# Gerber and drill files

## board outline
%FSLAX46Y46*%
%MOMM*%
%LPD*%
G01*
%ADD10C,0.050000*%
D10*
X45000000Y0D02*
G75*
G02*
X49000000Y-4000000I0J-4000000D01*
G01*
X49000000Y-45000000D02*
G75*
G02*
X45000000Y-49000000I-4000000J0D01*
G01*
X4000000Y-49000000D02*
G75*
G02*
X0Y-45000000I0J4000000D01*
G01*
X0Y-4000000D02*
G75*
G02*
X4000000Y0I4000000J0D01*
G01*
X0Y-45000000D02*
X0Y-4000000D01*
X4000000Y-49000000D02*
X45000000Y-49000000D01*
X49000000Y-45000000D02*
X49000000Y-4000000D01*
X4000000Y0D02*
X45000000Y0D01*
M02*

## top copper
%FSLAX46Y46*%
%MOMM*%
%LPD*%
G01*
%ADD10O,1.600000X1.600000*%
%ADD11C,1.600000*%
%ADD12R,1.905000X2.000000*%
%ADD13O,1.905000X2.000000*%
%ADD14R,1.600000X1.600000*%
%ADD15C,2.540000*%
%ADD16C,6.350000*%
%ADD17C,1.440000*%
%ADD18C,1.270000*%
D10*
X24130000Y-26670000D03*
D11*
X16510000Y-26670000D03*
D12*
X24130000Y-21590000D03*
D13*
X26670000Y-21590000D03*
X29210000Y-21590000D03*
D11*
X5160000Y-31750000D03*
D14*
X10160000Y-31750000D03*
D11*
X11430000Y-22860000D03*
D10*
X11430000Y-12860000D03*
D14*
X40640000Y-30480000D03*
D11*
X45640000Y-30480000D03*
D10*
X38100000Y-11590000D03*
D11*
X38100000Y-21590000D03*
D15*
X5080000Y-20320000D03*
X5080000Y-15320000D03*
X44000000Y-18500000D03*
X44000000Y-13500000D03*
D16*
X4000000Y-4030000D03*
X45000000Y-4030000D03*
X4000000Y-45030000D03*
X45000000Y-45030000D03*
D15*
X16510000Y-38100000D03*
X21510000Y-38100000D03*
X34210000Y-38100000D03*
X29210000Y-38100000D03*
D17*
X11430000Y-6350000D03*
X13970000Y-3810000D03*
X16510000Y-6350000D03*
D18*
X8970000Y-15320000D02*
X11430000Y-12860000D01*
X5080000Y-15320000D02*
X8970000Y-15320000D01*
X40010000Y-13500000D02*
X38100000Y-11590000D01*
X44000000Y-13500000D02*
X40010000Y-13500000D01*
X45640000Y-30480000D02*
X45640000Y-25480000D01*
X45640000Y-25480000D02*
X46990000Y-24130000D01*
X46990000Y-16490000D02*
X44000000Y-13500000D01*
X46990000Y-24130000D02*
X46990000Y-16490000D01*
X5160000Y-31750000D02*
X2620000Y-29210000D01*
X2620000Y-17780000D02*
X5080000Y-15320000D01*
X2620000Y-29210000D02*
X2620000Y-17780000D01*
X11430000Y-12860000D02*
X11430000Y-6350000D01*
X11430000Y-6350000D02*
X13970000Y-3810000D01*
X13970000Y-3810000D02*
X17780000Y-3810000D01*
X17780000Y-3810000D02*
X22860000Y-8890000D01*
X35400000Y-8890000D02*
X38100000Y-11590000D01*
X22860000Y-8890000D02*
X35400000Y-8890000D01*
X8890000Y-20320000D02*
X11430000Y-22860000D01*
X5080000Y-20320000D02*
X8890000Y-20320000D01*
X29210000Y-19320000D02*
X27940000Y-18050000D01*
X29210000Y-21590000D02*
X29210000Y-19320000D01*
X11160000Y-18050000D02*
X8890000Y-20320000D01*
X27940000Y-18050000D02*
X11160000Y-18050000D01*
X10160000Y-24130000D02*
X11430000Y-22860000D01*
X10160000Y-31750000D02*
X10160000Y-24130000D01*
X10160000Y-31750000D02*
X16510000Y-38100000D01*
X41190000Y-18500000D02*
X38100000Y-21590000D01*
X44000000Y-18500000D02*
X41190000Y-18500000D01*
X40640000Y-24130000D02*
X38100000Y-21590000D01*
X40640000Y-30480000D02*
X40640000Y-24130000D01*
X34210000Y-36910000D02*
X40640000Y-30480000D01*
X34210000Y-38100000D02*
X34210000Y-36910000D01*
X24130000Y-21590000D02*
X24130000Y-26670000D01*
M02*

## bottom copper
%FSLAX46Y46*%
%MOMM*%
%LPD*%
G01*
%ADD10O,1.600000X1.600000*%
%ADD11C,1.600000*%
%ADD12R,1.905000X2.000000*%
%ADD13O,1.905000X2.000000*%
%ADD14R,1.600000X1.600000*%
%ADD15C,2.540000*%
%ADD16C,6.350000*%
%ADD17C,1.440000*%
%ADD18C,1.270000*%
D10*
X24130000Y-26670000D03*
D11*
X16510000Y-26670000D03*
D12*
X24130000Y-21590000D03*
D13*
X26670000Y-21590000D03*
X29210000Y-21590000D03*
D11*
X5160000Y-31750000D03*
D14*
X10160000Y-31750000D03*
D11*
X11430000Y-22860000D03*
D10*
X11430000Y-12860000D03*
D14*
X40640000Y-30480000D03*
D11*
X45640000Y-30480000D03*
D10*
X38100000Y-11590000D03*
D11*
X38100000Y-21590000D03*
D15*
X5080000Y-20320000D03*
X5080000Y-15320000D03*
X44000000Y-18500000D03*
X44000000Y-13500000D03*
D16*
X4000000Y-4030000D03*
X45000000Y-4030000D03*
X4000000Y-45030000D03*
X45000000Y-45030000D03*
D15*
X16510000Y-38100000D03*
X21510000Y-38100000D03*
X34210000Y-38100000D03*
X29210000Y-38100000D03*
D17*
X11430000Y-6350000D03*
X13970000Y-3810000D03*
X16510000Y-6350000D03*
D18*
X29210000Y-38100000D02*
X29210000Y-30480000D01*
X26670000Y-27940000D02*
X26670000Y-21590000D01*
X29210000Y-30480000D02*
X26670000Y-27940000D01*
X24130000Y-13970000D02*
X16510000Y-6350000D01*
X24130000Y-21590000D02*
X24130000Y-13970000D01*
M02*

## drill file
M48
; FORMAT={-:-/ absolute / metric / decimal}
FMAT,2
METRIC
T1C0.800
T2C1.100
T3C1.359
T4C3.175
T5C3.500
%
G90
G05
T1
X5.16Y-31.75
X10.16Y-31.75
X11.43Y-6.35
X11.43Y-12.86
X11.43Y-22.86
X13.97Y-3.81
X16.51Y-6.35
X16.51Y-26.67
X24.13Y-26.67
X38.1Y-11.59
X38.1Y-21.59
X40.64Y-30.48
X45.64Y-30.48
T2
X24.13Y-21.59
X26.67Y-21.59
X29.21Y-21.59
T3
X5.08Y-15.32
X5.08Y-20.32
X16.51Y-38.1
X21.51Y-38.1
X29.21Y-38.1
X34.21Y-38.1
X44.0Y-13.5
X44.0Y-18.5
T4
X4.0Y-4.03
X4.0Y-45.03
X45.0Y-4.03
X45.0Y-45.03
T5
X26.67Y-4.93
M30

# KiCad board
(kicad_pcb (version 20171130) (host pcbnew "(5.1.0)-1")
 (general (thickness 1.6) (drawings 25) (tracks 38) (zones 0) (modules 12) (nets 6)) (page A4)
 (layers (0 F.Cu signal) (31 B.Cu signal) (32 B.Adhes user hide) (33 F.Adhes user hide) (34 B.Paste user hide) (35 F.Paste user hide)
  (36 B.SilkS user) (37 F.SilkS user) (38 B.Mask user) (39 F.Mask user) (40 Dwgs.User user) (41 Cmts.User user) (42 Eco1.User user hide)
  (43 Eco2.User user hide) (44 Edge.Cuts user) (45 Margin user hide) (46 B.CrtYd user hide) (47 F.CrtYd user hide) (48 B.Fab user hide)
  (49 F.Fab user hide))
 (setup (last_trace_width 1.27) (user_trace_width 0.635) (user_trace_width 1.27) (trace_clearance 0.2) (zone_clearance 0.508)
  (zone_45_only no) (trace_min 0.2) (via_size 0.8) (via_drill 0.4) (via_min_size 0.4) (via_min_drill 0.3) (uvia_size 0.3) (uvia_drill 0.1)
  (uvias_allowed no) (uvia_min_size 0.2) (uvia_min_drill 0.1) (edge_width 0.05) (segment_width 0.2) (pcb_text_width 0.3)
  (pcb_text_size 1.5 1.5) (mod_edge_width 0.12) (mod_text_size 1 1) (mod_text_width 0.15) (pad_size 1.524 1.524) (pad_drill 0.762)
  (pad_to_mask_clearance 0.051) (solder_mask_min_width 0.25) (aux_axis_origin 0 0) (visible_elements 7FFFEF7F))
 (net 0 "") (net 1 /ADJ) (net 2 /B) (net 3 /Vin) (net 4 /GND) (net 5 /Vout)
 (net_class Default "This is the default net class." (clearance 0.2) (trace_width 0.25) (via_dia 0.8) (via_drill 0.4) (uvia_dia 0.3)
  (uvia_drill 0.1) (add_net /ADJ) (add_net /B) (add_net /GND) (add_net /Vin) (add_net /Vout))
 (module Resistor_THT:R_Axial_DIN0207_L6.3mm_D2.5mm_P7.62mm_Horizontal (layer F.Cu) (at 16.51 26.67)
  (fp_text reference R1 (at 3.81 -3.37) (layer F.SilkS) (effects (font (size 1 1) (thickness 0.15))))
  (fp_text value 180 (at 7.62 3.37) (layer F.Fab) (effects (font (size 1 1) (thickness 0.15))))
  (pad 2 thru_hole oval (at 7.62 0) (size 1.6 1.6) (drill 0.8) (layers *.Cu *.Mask) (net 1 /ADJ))
  (pad 1 thru_hole circle (at 0 0) (size 1.6 1.6) (drill 0.8) (layers *.Cu *.Mask) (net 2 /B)))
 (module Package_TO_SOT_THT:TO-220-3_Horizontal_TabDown (layer F.Cu) (at 24.13 21.59)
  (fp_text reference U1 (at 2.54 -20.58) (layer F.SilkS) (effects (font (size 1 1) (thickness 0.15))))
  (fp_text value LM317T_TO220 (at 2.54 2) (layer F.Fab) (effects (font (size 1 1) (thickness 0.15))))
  (pad "" np_thru_hole oval (at 2.54 -16.66) (size 3.5 3.5) (drill 3.5) (layers *.Cu *.Mask))
  (pad 1 thru_hole rect (at 0 0) (size 1.905 2) (drill 1.1) (layers *.Cu *.Mask) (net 1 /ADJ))
  (pad 2 thru_hole oval (at 2.54 0) (size 1.905 2) (drill 1.1) (layers *.Cu *.Mask) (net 2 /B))
  (pad 3 thru_hole oval (at 5.08 0) (size 1.905 2) (drill 1.1) (layers *.Cu *.Mask) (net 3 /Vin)))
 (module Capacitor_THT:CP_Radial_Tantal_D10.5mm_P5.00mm (layer F.Cu) (at 10.16 31.75 180)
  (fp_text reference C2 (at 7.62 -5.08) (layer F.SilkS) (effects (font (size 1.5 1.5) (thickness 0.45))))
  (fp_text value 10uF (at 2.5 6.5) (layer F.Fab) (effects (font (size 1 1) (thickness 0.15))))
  (pad 2 thru_hole circle (at 5 0 180) (size 1.6 1.6) (drill 0.8) (layers *.Cu *.Mask) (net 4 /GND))
  (pad 1 thru_hole rect (at 0 0 180) (size 1.6 1.6) (drill 0.8) (layers *.Cu *.Mask) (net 3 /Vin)))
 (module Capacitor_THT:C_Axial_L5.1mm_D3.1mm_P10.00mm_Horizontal (layer F.Cu) (at 11.43 22.86 90)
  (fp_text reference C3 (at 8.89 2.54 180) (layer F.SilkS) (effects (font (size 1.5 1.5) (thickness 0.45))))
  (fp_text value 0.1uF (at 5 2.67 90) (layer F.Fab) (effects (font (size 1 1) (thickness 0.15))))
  (pad 1 thru_hole circle (at 0 0 90) (size 1.6 1.6) (drill 0.8) (layers *.Cu *.Mask) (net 3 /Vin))
  (pad 2 thru_hole oval (at 10 0 90) (size 1.6 1.6) (drill 0.8) (layers *.Cu *.Mask) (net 4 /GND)))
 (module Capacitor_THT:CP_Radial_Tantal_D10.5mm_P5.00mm (layer F.Cu) (at 40.64 30.48)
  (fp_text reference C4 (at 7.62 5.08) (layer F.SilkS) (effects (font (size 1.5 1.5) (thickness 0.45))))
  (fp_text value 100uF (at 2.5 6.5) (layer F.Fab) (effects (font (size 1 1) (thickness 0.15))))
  (pad 1 thru_hole rect (at 0 0) (size 1.6 1.6) (drill 0.8) (layers *.Cu *.Mask) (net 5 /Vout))
  (pad 2 thru_hole circle (at 5 0) (size 1.6 1.6) (drill 0.8) (layers *.Cu *.Mask) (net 4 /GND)))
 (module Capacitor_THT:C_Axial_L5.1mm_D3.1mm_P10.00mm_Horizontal (layer F.Cu) (at 38.1 21.59 90)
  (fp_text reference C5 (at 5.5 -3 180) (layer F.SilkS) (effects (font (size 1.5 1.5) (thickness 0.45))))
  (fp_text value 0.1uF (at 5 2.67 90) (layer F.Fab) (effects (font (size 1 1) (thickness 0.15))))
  (pad 2 thru_hole oval (at 10 0 90) (size 1.6 1.6) (drill 0.8) (layers *.Cu *.Mask) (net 4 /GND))
  (pad 1 thru_hole circle (at 0 0 90) (size 1.6 1.6) (drill 0.8) (layers *.Cu *.Mask) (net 5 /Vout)))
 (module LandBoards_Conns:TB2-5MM (layer F.Cu) (at 5.08 20.32 90)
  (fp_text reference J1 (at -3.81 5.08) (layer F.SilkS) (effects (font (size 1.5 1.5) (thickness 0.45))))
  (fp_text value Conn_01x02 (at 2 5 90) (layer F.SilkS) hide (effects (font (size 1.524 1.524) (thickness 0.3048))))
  (pad 1 thru_hole circle (at 0 0 90) (size 2.54 2.54) (drill 1.3589) (layers *.Cu *.Mask F.SilkS) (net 3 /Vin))
  (pad 2 thru_hole circle (at 5 0 90) (size 2.54 2.54) (drill 1.3589) (layers *.Cu *.Mask F.SilkS) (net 4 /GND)))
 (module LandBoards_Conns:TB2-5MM (layer F.Cu) (at 44 13.5 270)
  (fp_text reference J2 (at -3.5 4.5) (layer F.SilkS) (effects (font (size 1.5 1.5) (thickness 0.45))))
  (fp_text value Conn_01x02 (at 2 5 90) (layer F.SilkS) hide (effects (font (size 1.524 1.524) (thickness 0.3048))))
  (pad 2 thru_hole circle (at 5 0 270) (size 2.54 2.54) (drill 1.3589) (layers *.Cu *.Mask F.SilkS) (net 5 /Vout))
  (pad 1 thru_hole circle (at 0 0 270) (size 2.54 2.54) (drill 1.3589) (layers *.Cu *.Mask F.SilkS) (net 4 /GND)))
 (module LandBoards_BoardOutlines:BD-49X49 (layer F.Cu) (at 0 49.03)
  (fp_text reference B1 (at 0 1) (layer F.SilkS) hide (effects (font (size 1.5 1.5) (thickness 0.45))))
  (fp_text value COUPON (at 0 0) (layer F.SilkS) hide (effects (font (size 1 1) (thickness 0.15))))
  (pad 1 thru_hole circle (at 4 -45) (size 6.35 6.35) (drill 3.175) (layers *.Cu *.Mask F.SilkS))
  (pad 2 thru_hole circle (at 45 -45) (size 6.35 6.35) (drill 3.175) (layers *.Cu *.Mask F.SilkS))
  (pad 3 thru_hole circle (at 4 -4) (size 6.35 6.35) (drill 3.175) (layers *.Cu *.Mask F.SilkS))
  (pad 4 thru_hole circle (at 45 -4) (size 6.35 6.35) (drill 3.175) (layers *.Cu *.Mask F.SilkS)))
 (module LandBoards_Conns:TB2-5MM (layer F.Cu) (at 16.51 38.1)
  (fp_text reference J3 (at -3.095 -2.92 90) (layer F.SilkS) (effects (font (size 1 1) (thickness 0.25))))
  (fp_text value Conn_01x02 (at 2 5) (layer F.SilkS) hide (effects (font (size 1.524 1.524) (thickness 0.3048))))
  (pad 1 thru_hole circle (at 0 0) (size 2.54 2.54) (drill 1.3589) (layers *.Cu *.Mask F.SilkS) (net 3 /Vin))
  (pad 2 thru_hole circle (at 5 0) (size 2.54 2.54) (drill 1.3589) (layers *.Cu *.Mask F.SilkS)))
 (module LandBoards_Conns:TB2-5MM (layer F.Cu) (at 29.21 38.1)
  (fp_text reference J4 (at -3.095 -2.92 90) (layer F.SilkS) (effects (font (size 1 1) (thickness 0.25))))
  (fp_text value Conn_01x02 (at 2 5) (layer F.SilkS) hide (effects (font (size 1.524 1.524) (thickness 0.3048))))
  (pad 2 thru_hole circle (at 5 0) (size 2.54 2.54) (drill 1.3589) (layers *.Cu *.Mask F.SilkS) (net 5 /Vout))
  (pad 1 thru_hole circle (at 0 0) (size 2.54 2.54) (drill 1.3589) (layers *.Cu *.Mask F.SilkS) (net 2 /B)))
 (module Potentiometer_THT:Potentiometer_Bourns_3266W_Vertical (layer F.Cu) (at 11.43 6.35 180)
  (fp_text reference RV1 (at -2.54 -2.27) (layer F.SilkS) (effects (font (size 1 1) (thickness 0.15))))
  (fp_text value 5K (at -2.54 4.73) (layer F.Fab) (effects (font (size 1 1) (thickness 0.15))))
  (pad 1 thru_hole circle (at 0 0 180) (size 1.44 1.44) (drill 0.8) (layers *.Cu *.Mask) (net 4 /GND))
  (pad 2 thru_hole circle (at -2.54 2.54 180) (size 1.44 1.44) (drill 0.8) (layers *.Cu *.Mask) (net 4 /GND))
  (pad 3 thru_hole circle (at -5.08 0 180) (size 1.44 1.44) (drill 0.8) (layers *.Cu *.Mask) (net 1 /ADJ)))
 (gr_arc (start 45 4) (end 49 4) (angle -90) (layer Edge.Cuts) (width 0.05))
 (gr_arc (start 45 45) (end 45 49) (angle -90) (layer Edge.Cuts) (width 0.05))
 (gr_arc (start 4 45) (end 0 45) (angle -90) (layer Edge.Cuts) (width 0.05))
 (gr_arc (start 4 4) (end 4 0) (angle -90) (layer Edge.Cuts) (width 0.05))
 (gr_line (start 0 45) (end 0 4) (layer Edge.Cuts) (width 0.05))
 (gr_line (start 4 49) (end 45 49) (layer Edge.Cuts) (width 0.05))
 (gr_line (start 49 45) (end 49 4) (layer Edge.Cuts) (width 0.05))
 (gr_line (start 4 0) (end 45 0) (layer Edge.Cuts) (width 0.05))
 (segment (start 8.97 15.32) (end 11.43 12.86) (width 1.27) (layer F.Cu) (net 4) (status 20))
 (segment (start 5.08 15.32) (end 8.97 15.32) (width 1.27) (layer F.Cu) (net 4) (status 10))
 (segment (start 40.01 13.5) (end 38.1 11.59) (width 1.27) (layer F.Cu) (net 4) (status 20))
 (segment (start 44 13.5) (end 40.01 13.5) (width 1.27) (layer F.Cu) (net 4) (status 10))
 (segment (start 45.64 30.48) (end 45.64 25.48) (width 1.27) (layer F.Cu) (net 4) (status 10))
 (segment (start 45.64 25.48) (end 46.99 24.13) (width 1.27) (layer F.Cu) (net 4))
 (segment (start 46.99 16.49) (end 44 13.5) (width 1.27) (layer F.Cu) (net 4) (status 20))
 (segment (start 46.99 24.13) (end 46.99 16.49) (width 1.27) (layer F.Cu) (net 4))
 (segment (start 5.16 31.75) (end 2.62 29.21) (width 1.27) (layer F.Cu) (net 4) (status 10))
 (segment (start 2.62 17.78) (end 5.08 15.32) (width 1.27) (layer F.Cu) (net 4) (status 20))
 (segment (start 2.62 29.21) (end 2.62 17.78) (width 1.27) (layer F.Cu) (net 4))
 (segment (start 11.43 12.86) (end 11.43 6.35) (width 1.27) (layer F.Cu) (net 4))
 (segment (start 11.43 6.35) (end 13.97 3.81) (width 1.27) (layer F.Cu) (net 4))
 (segment (start 13.97 3.81) (end 17.78 3.81) (width 1.27) (layer F.Cu) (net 4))
 (segment (start 17.78 3.81) (end 22.86 8.89) (width 1.27) (layer F.Cu) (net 4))
 (segment (start 35.4 8.89) (end 38.1 11.59) (width 1.27) (layer F.Cu) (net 4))
 (segment (start 22.86 8.89) (end 35.4 8.89) (width 1.27) (layer F.Cu) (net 4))
 (segment (start 8.89 20.32) (end 11.43 22.86) (width 1.27) (layer F.Cu) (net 3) (status 20))
 (segment (start 5.08 20.32) (end 8.89 20.32) (width 1.27) (layer F.Cu) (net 3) (status 10))
 (segment (start 29.21 19.32) (end 27.94 18.05) (width 1.27) (layer F.Cu) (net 3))
 (segment (start 29.21 21.59) (end 29.21 19.32) (width 1.27) (layer F.Cu) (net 3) (status 10))
 (segment (start 11.16 18.05) (end 8.89 20.32) (width 1.27) (layer F.Cu) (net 3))
 (segment (start 27.94 18.05) (end 11.16 18.05) (width 1.27) (layer F.Cu) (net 3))
 (segment (start 10.16 24.13) (end 11.43 22.86) (width 1.27) (layer F.Cu) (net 3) (status 20))
 (segment (start 10.16 31.75) (end 10.16 24.13) (width 1.27) (layer F.Cu) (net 3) (status 10))
 (segment (start 10.16 31.75) (end 16.51 38.1) (width 1.27) (layer F.Cu) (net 3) (status 30))
 (segment (start 41.19 18.5) (end 38.1 21.59) (width 1.27) (layer F.Cu) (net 5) (status 20))
 (segment (start 44 18.5) (end 41.19 18.5) (width 1.27) (layer F.Cu) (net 5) (status 10))
 (segment (start 40.64 24.13) (end 38.1 21.59) (width 1.27) (layer F.Cu) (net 5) (status 20))
 (segment (start 40.64 30.48) (end 40.64 24.13) (width 1.27) (layer F.Cu) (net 5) (status 10))
 (segment (start 34.21 36.91) (end 40.64 30.48) (width 1.27) (layer F.Cu) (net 5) (status 30))
 (segment (start 34.21 38.1) (end 34.21 36.91) (width 1.27) (layer F.Cu) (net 5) (status 30))
 (segment (start 29.21 38.1) (end 29.21 30.48) (width 1.27) (layer B.Cu) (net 2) (status 10))
 (segment (start 26.67 27.94) (end 26.67 21.59) (width 1.27) (layer B.Cu) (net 2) (status 20))
 (segment (start 29.21 30.48) (end 26.67 27.94) (width 1.27) (layer B.Cu) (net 2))
 (segment (start 24.13 21.59) (end 24.13 26.67) (width 1.27) (layer F.Cu) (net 1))
 (segment (start 24.13 13.97) (end 16.51 6.35) (width 1.27) (layer B.Cu) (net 1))
 (segment (start 24.13 21.59) (end 24.13 13.97) (width 1.27) (layer B.Cu) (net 1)))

